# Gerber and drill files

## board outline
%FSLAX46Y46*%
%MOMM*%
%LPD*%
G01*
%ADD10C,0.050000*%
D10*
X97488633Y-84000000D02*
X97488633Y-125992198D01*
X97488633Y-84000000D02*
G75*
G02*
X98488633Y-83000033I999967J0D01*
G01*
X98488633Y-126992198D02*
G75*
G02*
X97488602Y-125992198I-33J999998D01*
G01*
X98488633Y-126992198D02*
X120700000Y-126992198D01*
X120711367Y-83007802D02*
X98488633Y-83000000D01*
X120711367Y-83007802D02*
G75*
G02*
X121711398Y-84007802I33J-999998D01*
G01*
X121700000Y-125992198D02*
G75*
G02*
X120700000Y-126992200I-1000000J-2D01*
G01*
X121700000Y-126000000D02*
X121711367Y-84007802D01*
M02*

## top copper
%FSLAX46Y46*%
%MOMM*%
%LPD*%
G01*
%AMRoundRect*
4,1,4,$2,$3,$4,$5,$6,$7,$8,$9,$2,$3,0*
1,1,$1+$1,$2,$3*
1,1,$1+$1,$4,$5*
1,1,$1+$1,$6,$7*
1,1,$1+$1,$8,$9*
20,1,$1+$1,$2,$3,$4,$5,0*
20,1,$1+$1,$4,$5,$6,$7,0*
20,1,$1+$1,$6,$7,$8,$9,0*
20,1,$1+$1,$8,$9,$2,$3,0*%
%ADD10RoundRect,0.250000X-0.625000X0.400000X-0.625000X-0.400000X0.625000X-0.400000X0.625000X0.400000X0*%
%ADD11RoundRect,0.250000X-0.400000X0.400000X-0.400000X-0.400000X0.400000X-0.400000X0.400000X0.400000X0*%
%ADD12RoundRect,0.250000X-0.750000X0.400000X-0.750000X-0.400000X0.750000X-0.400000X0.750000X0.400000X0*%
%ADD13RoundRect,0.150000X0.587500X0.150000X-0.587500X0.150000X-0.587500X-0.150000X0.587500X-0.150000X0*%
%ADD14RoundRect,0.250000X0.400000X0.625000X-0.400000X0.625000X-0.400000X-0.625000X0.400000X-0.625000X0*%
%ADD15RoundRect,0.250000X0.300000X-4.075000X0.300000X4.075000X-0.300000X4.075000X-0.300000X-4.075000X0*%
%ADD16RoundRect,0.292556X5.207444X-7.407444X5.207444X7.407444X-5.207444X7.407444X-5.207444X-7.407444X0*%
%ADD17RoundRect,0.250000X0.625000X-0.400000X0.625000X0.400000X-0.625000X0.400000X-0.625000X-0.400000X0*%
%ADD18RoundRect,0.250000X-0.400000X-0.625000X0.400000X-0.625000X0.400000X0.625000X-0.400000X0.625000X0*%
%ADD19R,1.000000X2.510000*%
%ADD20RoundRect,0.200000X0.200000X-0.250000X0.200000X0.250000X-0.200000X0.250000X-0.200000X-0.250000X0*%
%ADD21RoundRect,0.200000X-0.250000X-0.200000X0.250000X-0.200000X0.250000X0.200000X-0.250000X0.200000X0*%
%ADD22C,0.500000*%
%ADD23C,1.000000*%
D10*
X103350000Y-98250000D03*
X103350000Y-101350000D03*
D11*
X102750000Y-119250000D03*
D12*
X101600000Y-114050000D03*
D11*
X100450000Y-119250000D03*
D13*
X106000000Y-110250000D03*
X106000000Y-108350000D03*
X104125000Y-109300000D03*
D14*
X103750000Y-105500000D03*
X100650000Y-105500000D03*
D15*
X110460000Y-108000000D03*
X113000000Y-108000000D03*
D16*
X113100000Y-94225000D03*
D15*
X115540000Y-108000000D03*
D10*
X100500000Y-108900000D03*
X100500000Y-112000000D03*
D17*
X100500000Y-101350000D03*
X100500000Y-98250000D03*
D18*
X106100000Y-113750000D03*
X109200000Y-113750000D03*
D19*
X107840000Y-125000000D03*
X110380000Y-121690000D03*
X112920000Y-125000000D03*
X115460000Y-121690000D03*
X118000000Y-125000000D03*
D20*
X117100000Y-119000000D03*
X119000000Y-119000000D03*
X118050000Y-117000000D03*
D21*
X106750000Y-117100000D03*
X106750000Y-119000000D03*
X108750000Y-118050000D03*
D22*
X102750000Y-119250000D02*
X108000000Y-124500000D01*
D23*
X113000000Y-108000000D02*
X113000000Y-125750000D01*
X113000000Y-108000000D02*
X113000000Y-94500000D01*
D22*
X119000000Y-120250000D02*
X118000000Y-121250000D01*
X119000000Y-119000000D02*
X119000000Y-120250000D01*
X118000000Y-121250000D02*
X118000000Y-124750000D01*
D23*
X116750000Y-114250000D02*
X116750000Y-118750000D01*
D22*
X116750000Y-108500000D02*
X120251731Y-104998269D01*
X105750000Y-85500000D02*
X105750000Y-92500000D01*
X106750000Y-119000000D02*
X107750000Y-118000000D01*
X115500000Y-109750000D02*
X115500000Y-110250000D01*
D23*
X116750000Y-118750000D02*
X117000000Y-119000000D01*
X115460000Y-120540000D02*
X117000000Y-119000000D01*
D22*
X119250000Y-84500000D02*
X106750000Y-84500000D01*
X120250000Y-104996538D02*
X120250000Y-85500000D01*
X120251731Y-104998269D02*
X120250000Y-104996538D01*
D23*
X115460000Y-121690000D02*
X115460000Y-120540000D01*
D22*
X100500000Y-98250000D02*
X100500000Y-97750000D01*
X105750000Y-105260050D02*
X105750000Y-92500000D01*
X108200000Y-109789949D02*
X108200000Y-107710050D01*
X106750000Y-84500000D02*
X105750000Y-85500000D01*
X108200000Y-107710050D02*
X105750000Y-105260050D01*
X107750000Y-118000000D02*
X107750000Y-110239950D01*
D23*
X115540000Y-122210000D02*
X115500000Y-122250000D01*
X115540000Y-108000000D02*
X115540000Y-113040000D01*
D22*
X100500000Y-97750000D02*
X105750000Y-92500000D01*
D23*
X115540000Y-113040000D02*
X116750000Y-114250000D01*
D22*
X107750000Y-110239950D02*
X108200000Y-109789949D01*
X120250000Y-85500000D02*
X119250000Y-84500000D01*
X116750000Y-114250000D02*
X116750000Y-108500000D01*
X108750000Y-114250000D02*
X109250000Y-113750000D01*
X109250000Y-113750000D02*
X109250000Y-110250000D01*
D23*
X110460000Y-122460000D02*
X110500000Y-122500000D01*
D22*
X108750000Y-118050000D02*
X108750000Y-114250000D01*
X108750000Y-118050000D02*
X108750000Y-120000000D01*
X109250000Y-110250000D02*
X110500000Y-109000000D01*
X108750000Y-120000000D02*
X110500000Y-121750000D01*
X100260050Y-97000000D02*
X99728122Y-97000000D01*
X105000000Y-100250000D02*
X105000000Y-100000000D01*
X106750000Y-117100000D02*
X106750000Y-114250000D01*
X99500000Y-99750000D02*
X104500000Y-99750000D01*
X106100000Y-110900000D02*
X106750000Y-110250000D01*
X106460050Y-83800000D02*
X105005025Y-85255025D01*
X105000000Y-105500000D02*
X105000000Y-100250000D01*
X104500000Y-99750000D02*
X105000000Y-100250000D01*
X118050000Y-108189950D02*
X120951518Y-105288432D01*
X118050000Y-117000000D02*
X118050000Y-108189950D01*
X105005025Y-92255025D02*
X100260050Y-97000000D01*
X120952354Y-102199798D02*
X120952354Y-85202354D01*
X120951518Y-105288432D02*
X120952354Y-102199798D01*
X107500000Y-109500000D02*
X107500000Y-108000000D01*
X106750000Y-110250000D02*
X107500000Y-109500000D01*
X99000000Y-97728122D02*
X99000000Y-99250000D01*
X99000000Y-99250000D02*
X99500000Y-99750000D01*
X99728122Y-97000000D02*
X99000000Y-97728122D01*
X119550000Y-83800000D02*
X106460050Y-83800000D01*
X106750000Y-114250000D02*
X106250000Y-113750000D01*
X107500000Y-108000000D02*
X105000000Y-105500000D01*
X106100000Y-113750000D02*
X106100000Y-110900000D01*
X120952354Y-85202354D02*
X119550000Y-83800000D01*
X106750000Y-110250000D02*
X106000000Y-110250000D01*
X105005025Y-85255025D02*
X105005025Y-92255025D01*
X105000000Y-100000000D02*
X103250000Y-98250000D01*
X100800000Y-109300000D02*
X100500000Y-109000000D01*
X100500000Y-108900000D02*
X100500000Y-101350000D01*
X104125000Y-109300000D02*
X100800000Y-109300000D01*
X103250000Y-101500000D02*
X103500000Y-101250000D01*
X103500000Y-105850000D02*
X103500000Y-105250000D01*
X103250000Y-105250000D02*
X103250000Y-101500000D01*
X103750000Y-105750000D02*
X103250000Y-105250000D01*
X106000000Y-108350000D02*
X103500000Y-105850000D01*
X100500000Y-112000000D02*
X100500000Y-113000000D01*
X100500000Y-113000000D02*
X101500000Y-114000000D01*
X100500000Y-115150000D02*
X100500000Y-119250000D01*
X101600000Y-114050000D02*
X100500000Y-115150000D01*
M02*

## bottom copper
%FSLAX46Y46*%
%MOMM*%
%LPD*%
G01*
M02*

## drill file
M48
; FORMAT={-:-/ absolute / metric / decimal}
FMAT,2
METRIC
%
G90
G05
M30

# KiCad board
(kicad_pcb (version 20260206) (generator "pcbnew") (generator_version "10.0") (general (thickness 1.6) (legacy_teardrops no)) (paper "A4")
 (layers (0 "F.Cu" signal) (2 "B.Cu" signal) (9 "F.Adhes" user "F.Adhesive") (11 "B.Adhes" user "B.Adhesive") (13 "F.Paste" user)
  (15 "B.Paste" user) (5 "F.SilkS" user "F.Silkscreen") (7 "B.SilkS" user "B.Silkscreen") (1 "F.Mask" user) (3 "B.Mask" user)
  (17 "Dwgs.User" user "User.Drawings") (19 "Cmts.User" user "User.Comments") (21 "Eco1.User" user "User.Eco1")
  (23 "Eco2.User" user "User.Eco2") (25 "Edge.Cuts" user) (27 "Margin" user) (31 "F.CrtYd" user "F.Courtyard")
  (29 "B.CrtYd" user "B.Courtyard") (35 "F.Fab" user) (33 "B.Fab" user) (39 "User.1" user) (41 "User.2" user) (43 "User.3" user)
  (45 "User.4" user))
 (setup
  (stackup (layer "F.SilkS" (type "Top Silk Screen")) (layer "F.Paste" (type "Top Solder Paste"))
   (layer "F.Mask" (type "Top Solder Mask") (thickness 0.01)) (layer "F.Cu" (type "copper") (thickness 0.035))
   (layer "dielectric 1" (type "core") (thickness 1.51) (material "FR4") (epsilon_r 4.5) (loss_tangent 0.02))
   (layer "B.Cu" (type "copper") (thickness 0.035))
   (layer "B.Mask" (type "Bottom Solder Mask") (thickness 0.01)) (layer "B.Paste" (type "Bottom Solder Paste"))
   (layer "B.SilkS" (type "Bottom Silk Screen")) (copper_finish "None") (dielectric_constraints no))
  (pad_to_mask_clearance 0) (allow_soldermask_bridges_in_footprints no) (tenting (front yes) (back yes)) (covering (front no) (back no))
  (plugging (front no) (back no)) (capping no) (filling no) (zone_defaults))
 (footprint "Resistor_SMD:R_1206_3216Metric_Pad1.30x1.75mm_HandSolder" (layer "F.Cu") (at 103.35 99.8 -90)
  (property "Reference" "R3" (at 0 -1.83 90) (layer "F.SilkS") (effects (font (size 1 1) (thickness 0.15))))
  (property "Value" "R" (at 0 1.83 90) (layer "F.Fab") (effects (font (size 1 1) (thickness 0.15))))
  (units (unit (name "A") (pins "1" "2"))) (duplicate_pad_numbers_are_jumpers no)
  (pad "1" smd roundrect (at -1.55 0 270) (size 1.3 1.75) (layers "F.Cu" "F.Mask" "F.Paste") (roundrect_rratio 0.192308) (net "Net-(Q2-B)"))
  (pad "2" smd roundrect (at 1.55 0 270) (size 1.3 1.75) (layers "F.Cu" "F.Mask" "F.Paste") (roundrect_rratio 0.192308) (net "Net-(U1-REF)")))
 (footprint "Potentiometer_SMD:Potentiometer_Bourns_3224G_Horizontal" (layer "F.Cu") (at 101.6 116.65 -90)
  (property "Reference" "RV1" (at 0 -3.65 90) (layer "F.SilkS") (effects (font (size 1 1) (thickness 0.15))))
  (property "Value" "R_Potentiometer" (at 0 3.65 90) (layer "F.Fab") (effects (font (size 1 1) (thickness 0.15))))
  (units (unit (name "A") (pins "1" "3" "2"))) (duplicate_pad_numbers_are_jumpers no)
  (pad "1" smd roundrect (at 2.6 -1.15 270) (size 1.3 1.3) (layers "F.Cu" "F.Mask" "F.Paste") (roundrect_rratio 0.192308) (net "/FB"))
  (pad "2" smd roundrect (at -2.6 0 270) (size 1.3 2) (layers "F.Cu" "F.Mask" "F.Paste") (roundrect_rratio 0.192308) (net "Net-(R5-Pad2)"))
  (pad "3" smd roundrect (at 2.6 1.15 270) (size 1.3 1.3) (layers "F.Cu" "F.Mask" "F.Paste") (roundrect_rratio 0.192308)
   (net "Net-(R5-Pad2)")))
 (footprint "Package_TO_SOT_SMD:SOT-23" (layer "F.Cu") (at 105.0625 109.3 180)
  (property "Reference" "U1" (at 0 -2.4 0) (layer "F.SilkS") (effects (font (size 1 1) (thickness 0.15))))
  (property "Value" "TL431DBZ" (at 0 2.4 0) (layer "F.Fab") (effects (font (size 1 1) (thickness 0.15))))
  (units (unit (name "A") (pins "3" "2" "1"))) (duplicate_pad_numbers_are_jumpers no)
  (pad "1" smd roundrect (at -0.9375 -0.95 180) (size 1.475 0.6) (layers "F.Cu" "F.Mask" "F.Paste") (roundrect_rratio 0.25)
   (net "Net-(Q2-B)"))
  (pad "2" smd roundrect (at -0.9375 0.95 180) (size 1.475 0.6) (layers "F.Cu" "F.Mask" "F.Paste") (roundrect_rratio 0.25)
   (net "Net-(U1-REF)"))
  (pad "3" smd roundrect (at 0.9375 0 180) (size 1.475 0.6) (layers "F.Cu" "F.Mask" "F.Paste") (roundrect_rratio 0.25) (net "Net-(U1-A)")))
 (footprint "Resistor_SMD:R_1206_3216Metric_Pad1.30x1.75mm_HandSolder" (layer "F.Cu") (at 102.2 105.5 180)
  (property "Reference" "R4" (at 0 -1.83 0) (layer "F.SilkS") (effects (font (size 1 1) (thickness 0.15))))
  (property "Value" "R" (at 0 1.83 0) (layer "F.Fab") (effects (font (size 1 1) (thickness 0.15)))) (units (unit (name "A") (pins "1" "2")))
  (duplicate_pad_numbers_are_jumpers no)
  (pad "1" smd roundrect (at -1.55 0 180) (size 1.3 1.75) (layers "F.Cu" "F.Mask" "F.Paste") (roundrect_rratio 0.192308)
   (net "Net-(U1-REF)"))
  (pad "2" smd roundrect (at 1.55 0 180) (size 1.3 1.75) (layers "F.Cu" "F.Mask" "F.Paste") (roundrect_rratio 0.192308) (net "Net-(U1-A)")))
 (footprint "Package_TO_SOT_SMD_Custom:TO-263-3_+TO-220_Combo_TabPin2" (layer "F.Cu") (at 113 98.325 90)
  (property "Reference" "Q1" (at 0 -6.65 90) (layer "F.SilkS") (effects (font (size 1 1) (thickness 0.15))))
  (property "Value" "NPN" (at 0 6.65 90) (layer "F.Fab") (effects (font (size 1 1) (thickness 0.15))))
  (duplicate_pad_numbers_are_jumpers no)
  (pad "" smd roundrect (at -0.925 -2.775 90) (size 4.55 5.25) (layers "F.Paste") (roundrect_rratio 0.054945))
  (pad "" smd roundrect (at -0.925 2.775 90) (size 4.55 5.25) (layers "F.Paste") (roundrect_rratio 0.054945))
  (pad "" smd roundrect (at 3.925 -2.775 90) (size 4.55 5.25) (layers "F.Paste") (roundrect_rratio 0.054945))
  (pad "" smd roundrect (at 3.925 2.775 90) (size 4.55 5.25) (layers "F.Paste") (roundrect_rratio 0.054945))
  (pad "" smd roundrect (at 9 -2.775 90) (size 4.55 5.25) (layers "F.Paste") (roundrect_rratio 0.054945))
  (pad "" smd roundrect (at 9 2.775 90) (size 4.55 5.25) (layers "F.Paste") (roundrect_rratio 0.054945))
  (pad "1" smd roundrect (at -9.675 -2.54 90) (size 8.65 1.1) (layers "F.Cu" "F.Mask" "F.Paste") (roundrect_rratio 0.227273)
   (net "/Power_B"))
  (pad "2" smd roundrect (at -9.675 0 90) (size 8.65 1.1) (layers "F.Cu" "F.Mask" "F.Paste") (roundrect_rratio 0.227273) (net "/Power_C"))
  (pad "2" smd roundrect (at 4.1 0.1 90) (size 15.4 11) (layers "F.Cu" "F.Mask") (roundrect_rratio 0.026596) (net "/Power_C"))
  (pad "3" smd roundrect (at -9.675 2.54 90) (size 8.65 1.1) (layers "F.Cu" "F.Mask" "F.Paste") (roundrect_rratio 0.227273) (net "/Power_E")))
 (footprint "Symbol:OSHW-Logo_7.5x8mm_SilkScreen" (layer "F.Cu") (at 101.85 91.25)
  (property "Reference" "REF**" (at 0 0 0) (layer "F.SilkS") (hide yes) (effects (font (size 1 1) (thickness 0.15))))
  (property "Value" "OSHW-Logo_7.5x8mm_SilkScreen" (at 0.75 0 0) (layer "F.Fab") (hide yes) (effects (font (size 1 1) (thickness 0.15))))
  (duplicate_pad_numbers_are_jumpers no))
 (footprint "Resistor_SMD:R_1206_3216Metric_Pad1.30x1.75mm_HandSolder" (layer "F.Cu") (at 100.5 110.45 -90)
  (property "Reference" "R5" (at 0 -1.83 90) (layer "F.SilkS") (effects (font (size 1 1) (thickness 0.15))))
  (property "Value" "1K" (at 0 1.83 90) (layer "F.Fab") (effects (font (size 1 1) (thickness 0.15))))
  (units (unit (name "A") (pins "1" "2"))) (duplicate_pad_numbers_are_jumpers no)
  (pad "1" smd roundrect (at -1.55 0 270) (size 1.3 1.75) (layers "F.Cu" "F.Mask" "F.Paste") (roundrect_rratio 0.192308) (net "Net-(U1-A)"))
  (pad "2" smd roundrect (at 1.55 0 270) (size 1.3 1.75) (layers "F.Cu" "F.Mask" "F.Paste") (roundrect_rratio 0.192308)
   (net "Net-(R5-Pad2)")))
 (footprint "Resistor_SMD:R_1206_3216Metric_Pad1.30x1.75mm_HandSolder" (layer "F.Cu") (at 100.5 99.8 90)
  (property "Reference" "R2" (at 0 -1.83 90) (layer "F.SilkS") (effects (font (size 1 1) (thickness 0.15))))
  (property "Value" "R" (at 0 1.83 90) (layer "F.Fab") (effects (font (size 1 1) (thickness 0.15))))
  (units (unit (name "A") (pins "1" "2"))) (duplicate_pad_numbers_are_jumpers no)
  (pad "1" smd roundrect (at -1.55 0 90) (size 1.3 1.75) (layers "F.Cu" "F.Mask" "F.Paste") (roundrect_rratio 0.192308) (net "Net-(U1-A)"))
  (pad "2" smd roundrect (at 1.55 0 90) (size 1.3 1.75) (layers "F.Cu" "F.Mask" "F.Paste") (roundrect_rratio 0.192308) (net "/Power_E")))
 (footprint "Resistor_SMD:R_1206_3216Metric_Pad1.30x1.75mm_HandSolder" (layer "F.Cu") (at 107.65 113.75)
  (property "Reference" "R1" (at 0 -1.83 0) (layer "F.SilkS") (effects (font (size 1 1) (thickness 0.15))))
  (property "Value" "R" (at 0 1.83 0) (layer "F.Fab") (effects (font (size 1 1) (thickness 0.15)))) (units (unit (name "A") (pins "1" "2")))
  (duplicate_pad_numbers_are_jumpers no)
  (pad "1" smd roundrect (at -1.55 0) (size 1.3 1.75) (layers "F.Cu" "F.Mask" "F.Paste") (roundrect_rratio 0.192308) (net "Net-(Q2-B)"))
  (pad "2" smd roundrect (at 1.55 0) (size 1.3 1.75) (layers "F.Cu" "F.Mask" "F.Paste") (roundrect_rratio 0.192308) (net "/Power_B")))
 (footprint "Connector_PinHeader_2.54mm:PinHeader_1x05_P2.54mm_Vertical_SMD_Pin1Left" (layer "F.Cu") (at 112.92 123.345 90)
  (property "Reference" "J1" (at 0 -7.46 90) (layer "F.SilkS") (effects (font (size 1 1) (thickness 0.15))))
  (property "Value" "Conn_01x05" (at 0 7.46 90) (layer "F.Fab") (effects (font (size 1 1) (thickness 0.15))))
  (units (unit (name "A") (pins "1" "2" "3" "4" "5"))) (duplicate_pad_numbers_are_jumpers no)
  (pad "1" smd rect (at -1.655 -5.08 90) (size 2.51 1) (layers "F.Cu" "F.Mask" "F.Paste") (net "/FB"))
  (pad "2" smd rect (at 1.655 -2.54 90) (size 2.51 1) (layers "F.Cu" "F.Mask" "F.Paste") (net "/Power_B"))
  (pad "3" smd rect (at -1.655 0 90) (size 2.51 1) (layers "F.Cu" "F.Mask" "F.Paste") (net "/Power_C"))
  (pad "4" smd rect (at 1.655 2.54 90) (size 2.51 1) (layers "F.Cu" "F.Mask" "F.Paste") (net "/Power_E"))
  (pad "5" smd rect (at -1.655 5.08 90) (size 2.51 1) (layers "F.Cu" "F.Mask" "F.Paste") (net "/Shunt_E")))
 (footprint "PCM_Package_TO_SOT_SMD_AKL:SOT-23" (layer "F.Cu") (at 118.05 118 90)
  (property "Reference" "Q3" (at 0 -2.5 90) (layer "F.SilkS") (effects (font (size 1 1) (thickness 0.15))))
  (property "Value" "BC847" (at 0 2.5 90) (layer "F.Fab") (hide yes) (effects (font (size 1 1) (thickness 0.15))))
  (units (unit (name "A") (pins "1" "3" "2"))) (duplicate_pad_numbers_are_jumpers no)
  (pad "1" smd roundrect (at -1 -0.95 90) (size 0.9 0.8) (layers "F.Cu" "F.Mask" "F.Paste") (roundrect_rratio 0.25) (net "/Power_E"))
  (pad "2" smd roundrect (at -1 0.95 90) (size 0.9 0.8) (layers "F.Cu" "F.Mask" "F.Paste") (roundrect_rratio 0.25) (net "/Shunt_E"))
  (pad "3" smd roundrect (at 1 0 90) (size 0.9 0.8) (layers "F.Cu" "F.Mask" "F.Paste") (roundrect_rratio 0.25) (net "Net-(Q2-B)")))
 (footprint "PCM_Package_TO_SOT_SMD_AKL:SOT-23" (layer "F.Cu") (at 107.75 118.05)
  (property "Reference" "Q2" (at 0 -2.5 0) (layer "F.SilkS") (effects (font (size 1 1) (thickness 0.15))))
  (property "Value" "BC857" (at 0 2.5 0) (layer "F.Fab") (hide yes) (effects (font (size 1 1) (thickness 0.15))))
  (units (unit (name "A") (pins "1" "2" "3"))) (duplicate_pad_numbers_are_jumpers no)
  (pad "1" smd roundrect (at -1 -0.95) (size 0.9 0.8) (layers "F.Cu" "F.Mask" "F.Paste") (roundrect_rratio 0.25) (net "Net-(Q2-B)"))
  (pad "2" smd roundrect (at -1 0.95) (size 0.9 0.8) (layers "F.Cu" "F.Mask" "F.Paste") (roundrect_rratio 0.25) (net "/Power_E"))
  (pad "3" smd roundrect (at 1 0) (size 0.9 0.8) (layers "F.Cu" "F.Mask" "F.Paste") (roundrect_rratio 0.25) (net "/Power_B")))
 (gr_line (start 97.488633 84) (end 97.488633 125.992198) (stroke (width 0.05) (type default)) (layer "Edge.Cuts"))
 (gr_arc (start 97.488633 84) (mid 97.781526 83.292893) (end 98.488633 83) (stroke (width 0.05) (type default)) (layer "Edge.Cuts"))
 (gr_arc (start 98.488633 126.992198) (mid 97.781526 126.699305) (end 97.488633 125.992198) (stroke (width 0.05) (type default))
  (layer "Edge.Cuts"))
 (gr_line (start 98.488633 126.992198) (end 120.7 126.992198) (stroke (width 0.05) (type default)) (layer "Edge.Cuts"))
 (gr_line (start 120.711367 83.007802) (end 98.488633 83) (stroke (width 0.05) (type default)) (layer "Edge.Cuts"))
 (gr_arc (start 120.711367 83.007802) (mid 121.418474 83.300695) (end 121.711367 84.007802) (stroke (width 0.05) (type default))
  (layer "Edge.Cuts"))
 (gr_arc (start 121.7 125.992198) (mid 121.407107 126.699305) (end 120.7 126.992198) (stroke (width 0.05) (type default))
  (layer "Edge.Cuts"))
 (gr_line (start 121.7 126) (end 121.711367 84.007802) (stroke (width 0.05) (type default)) (layer "Edge.Cuts"))
 (segment (start 102.75 119.25) (end 108 124.5) (width 0.5) (layer "F.Cu") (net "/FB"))
 (segment (start 113 108) (end 113 125.75) (width 1) (layer "F.Cu") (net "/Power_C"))
 (segment (start 113 108) (end 113 94.5) (width 1) (layer "F.Cu") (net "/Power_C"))
 (segment (start 119 120.25) (end 118 121.25) (width 0.5) (layer "F.Cu") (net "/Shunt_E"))
 (segment (start 119 119) (end 119 120.25) (width 0.5) (layer "F.Cu") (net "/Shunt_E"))
 (segment (start 118 121.25) (end 118 124.75) (width 0.5) (layer "F.Cu") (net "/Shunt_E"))
 (segment (start 116.75 114.25) (end 116.75 118.75) (width 1) (layer "F.Cu") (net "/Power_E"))
 (segment (start 116.75 108.5) (end 120.251731 104.998269) (width 0.5) (layer "F.Cu") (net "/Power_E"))
 (segment (start 105.75 85.5) (end 105.75 92.5) (width 0.5) (layer "F.Cu") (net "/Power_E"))
 (segment (start 106.75 119) (end 107.75 118) (width 0.5) (layer "F.Cu") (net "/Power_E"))
 (segment (start 115.5 109.75) (end 115.5 110.25) (width 0.5) (layer "F.Cu") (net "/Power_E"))
 (segment (start 116.75 118.75) (end 117 119) (width 1) (layer "F.Cu") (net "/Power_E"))
 (segment (start 115.46 120.54) (end 117 119) (width 1) (layer "F.Cu") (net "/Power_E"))
 (segment (start 119.25 84.5) (end 106.75 84.5) (width 0.5) (layer "F.Cu") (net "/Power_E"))
 (segment (start 120.25 104.996538) (end 120.25 85.5) (width 0.5) (layer "F.Cu") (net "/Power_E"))
 (segment (start 120.251731 104.998269) (end 120.25 104.996538) (width 0.5) (layer "F.Cu") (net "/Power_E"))
 (segment (start 115.46 121.69) (end 115.46 120.54) (width 1) (layer "F.Cu") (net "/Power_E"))
 (segment (start 100.5 98.25) (end 100.5 97.75) (width 0.5) (layer "F.Cu") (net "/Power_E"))
 (segment (start 105.75 105.26005) (end 105.75 92.5) (width 0.5) (layer "F.Cu") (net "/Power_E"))
 (segment (start 108.2 109.789949) (end 108.2 107.71005) (width 0.5) (layer "F.Cu") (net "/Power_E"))
 (segment (start 106.75 84.5) (end 105.75 85.5) (width 0.5) (layer "F.Cu") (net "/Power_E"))
 (segment (start 108.2 107.71005) (end 105.75 105.26005) (width 0.5) (layer "F.Cu") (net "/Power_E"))
 (segment (start 107.75 118) (end 107.75 110.23995) (width 0.5) (layer "F.Cu") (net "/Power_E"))
 (segment (start 115.54 122.21) (end 115.5 122.25) (width 1) (layer "F.Cu") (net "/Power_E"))
 (segment (start 115.54 108) (end 115.54 113.04) (width 1) (layer "F.Cu") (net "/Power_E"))
 (segment (start 100.5 97.75) (end 105.75 92.5) (width 0.5) (layer "F.Cu") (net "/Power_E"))
 (segment (start 115.54 113.04) (end 116.75 114.25) (width 1) (layer "F.Cu") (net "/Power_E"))
 (segment (start 107.75 110.23995) (end 108.2 109.789949) (width 0.5) (layer "F.Cu") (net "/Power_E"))
 (segment (start 120.25 85.5) (end 119.25 84.5) (width 0.5) (layer "F.Cu") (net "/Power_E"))
 (segment (start 116.75 114.25) (end 116.75 108.5) (width 0.5) (layer "F.Cu") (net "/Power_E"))
 (segment (start 108.75 114.25) (end 109.25 113.75) (width 0.5) (layer "F.Cu") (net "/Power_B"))
 (segment (start 109.25 113.75) (end 109.25 110.25) (width 0.5) (layer "F.Cu") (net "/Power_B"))
 (segment (start 110.46 122.46) (end 110.5 122.5) (width 1) (layer "F.Cu") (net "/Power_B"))
 (segment (start 108.75 118.05) (end 108.75 114.25) (width 0.5) (layer "F.Cu") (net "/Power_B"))
 (segment (start 108.75 118.05) (end 108.75 120) (width 0.5) (layer "F.Cu") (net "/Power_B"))
 (segment (start 109.25 110.25) (end 110.5 109) (width 0.5) (layer "F.Cu") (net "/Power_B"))
 (segment (start 108.75 120) (end 110.5 121.75) (width 0.5) (layer "F.Cu") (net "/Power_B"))
 (segment (start 100.26005 97) (end 99.728122 97) (width 0.5) (layer "F.Cu") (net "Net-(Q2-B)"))
 (segment (start 105 100.25) (end 105 100) (width 0.5) (layer "F.Cu") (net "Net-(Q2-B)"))
 (segment (start 106.75 117.1) (end 106.75 114.25) (width 0.5) (layer "F.Cu") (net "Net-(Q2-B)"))
 (segment (start 99.5 99.75) (end 104.5 99.75) (width 0.5) (layer "F.Cu") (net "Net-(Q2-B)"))
 (segment (start 106.1 110.9) (end 106.75 110.25) (width 0.5) (layer "F.Cu") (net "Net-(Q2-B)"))
 (segment (start 106.46005 83.8) (end 105.005025 85.255025) (width 0.5) (layer "F.Cu") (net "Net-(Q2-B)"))
 (segment (start 105 105.5) (end 105 100.25) (width 0.5) (layer "F.Cu") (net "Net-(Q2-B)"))
 (segment (start 104.5 99.75) (end 105 100.25) (width 0.5) (layer "F.Cu") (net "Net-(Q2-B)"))
 (segment (start 118.05 108.18995) (end 120.951518 105.288432) (width 0.5) (layer "F.Cu") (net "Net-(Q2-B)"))
 (segment (start 118.05 117) (end 118.05 108.18995) (width 0.5) (layer "F.Cu") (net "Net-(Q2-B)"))
 (segment (start 105.005025 92.255025) (end 100.26005 97) (width 0.5) (layer "F.Cu") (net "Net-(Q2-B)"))
 (segment (start 120.952354 102.199798) (end 120.952354 85.202354) (width 0.5) (layer "F.Cu") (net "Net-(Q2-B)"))
 (segment (start 120.951518 105.288432) (end 120.952354 102.199798) (width 0.5) (layer "F.Cu") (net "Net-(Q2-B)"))
 (segment (start 107.5 109.5) (end 107.5 108) (width 0.5) (layer "F.Cu") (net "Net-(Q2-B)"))
 (segment (start 106.75 110.25) (end 107.5 109.5) (width 0.5) (layer "F.Cu") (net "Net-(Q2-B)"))
 (segment (start 99 97.728122) (end 99 99.25) (width 0.5) (layer "F.Cu") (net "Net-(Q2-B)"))
 (segment (start 99 99.25) (end 99.5 99.75) (width 0.5) (layer "F.Cu") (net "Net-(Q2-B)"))
 (segment (start 99.728122 97) (end 99 97.728122) (width 0.5) (layer "F.Cu") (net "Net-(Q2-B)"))
 (segment (start 119.55 83.8) (end 106.46005 83.8) (width 0.5) (layer "F.Cu") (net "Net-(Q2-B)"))
 (segment (start 106.75 114.25) (end 106.25 113.75) (width 0.5) (layer "F.Cu") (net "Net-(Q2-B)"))
 (segment (start 107.5 108) (end 105 105.5) (width 0.5) (layer "F.Cu") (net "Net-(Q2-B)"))
 (segment (start 106.1 113.75) (end 106.1 110.9) (width 0.5) (layer "F.Cu") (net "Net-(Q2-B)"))
 (segment (start 120.952354 85.202354) (end 119.55 83.8) (width 0.5) (layer "F.Cu") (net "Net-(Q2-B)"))
 (segment (start 106.75 110.25) (end 106 110.25) (width 0.5) (layer "F.Cu") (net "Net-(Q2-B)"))
 (segment (start 105.005025 85.255025) (end 105.005025 92.255025) (width 0.5) (layer "F.Cu") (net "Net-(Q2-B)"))
 (segment (start 105 100) (end 103.25 98.25) (width 0.5) (layer "F.Cu") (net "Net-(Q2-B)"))
 (segment (start 100.8 109.3) (end 100.5 109) (width 0.5) (layer "F.Cu") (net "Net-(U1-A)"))
 (segment (start 100.5 108.9) (end 100.5 101.35) (width 0.5) (layer "F.Cu") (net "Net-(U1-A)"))
 (segment (start 104.125 109.3) (end 100.8 109.3) (width 0.5) (layer "F.Cu") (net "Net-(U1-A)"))
 (segment (start 103.25 101.5) (end 103.5 101.25) (width 0.5) (layer "F.Cu") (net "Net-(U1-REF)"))
 (segment (start 103.5 105.85) (end 103.5 105.25) (width 0.5) (layer "F.Cu") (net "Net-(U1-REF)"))
 (segment (start 103.25 105.25) (end 103.25 101.5) (width 0.5) (layer "F.Cu") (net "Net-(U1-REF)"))
 (segment (start 103.75 105.75) (end 103.25 105.25) (width 0.5) (layer "F.Cu") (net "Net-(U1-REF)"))
 (segment (start 106 108.35) (end 103.5 105.85) (width 0.5) (layer "F.Cu") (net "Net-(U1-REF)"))
 (segment (start 100.5 112) (end 100.5 113) (width 0.5) (layer "F.Cu") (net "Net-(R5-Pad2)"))
 (segment (start 100.5 113) (end 101.5 114) (width 0.5) (layer "F.Cu") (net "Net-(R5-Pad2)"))
 (segment (start 100.5 115.15) (end 100.5 119.25) (width 0.5) (layer "F.Cu") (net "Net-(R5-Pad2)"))
 (segment (start 101.6 114.05) (end 100.5 115.15) (width 0.5) (layer "F.Cu") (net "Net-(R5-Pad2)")))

